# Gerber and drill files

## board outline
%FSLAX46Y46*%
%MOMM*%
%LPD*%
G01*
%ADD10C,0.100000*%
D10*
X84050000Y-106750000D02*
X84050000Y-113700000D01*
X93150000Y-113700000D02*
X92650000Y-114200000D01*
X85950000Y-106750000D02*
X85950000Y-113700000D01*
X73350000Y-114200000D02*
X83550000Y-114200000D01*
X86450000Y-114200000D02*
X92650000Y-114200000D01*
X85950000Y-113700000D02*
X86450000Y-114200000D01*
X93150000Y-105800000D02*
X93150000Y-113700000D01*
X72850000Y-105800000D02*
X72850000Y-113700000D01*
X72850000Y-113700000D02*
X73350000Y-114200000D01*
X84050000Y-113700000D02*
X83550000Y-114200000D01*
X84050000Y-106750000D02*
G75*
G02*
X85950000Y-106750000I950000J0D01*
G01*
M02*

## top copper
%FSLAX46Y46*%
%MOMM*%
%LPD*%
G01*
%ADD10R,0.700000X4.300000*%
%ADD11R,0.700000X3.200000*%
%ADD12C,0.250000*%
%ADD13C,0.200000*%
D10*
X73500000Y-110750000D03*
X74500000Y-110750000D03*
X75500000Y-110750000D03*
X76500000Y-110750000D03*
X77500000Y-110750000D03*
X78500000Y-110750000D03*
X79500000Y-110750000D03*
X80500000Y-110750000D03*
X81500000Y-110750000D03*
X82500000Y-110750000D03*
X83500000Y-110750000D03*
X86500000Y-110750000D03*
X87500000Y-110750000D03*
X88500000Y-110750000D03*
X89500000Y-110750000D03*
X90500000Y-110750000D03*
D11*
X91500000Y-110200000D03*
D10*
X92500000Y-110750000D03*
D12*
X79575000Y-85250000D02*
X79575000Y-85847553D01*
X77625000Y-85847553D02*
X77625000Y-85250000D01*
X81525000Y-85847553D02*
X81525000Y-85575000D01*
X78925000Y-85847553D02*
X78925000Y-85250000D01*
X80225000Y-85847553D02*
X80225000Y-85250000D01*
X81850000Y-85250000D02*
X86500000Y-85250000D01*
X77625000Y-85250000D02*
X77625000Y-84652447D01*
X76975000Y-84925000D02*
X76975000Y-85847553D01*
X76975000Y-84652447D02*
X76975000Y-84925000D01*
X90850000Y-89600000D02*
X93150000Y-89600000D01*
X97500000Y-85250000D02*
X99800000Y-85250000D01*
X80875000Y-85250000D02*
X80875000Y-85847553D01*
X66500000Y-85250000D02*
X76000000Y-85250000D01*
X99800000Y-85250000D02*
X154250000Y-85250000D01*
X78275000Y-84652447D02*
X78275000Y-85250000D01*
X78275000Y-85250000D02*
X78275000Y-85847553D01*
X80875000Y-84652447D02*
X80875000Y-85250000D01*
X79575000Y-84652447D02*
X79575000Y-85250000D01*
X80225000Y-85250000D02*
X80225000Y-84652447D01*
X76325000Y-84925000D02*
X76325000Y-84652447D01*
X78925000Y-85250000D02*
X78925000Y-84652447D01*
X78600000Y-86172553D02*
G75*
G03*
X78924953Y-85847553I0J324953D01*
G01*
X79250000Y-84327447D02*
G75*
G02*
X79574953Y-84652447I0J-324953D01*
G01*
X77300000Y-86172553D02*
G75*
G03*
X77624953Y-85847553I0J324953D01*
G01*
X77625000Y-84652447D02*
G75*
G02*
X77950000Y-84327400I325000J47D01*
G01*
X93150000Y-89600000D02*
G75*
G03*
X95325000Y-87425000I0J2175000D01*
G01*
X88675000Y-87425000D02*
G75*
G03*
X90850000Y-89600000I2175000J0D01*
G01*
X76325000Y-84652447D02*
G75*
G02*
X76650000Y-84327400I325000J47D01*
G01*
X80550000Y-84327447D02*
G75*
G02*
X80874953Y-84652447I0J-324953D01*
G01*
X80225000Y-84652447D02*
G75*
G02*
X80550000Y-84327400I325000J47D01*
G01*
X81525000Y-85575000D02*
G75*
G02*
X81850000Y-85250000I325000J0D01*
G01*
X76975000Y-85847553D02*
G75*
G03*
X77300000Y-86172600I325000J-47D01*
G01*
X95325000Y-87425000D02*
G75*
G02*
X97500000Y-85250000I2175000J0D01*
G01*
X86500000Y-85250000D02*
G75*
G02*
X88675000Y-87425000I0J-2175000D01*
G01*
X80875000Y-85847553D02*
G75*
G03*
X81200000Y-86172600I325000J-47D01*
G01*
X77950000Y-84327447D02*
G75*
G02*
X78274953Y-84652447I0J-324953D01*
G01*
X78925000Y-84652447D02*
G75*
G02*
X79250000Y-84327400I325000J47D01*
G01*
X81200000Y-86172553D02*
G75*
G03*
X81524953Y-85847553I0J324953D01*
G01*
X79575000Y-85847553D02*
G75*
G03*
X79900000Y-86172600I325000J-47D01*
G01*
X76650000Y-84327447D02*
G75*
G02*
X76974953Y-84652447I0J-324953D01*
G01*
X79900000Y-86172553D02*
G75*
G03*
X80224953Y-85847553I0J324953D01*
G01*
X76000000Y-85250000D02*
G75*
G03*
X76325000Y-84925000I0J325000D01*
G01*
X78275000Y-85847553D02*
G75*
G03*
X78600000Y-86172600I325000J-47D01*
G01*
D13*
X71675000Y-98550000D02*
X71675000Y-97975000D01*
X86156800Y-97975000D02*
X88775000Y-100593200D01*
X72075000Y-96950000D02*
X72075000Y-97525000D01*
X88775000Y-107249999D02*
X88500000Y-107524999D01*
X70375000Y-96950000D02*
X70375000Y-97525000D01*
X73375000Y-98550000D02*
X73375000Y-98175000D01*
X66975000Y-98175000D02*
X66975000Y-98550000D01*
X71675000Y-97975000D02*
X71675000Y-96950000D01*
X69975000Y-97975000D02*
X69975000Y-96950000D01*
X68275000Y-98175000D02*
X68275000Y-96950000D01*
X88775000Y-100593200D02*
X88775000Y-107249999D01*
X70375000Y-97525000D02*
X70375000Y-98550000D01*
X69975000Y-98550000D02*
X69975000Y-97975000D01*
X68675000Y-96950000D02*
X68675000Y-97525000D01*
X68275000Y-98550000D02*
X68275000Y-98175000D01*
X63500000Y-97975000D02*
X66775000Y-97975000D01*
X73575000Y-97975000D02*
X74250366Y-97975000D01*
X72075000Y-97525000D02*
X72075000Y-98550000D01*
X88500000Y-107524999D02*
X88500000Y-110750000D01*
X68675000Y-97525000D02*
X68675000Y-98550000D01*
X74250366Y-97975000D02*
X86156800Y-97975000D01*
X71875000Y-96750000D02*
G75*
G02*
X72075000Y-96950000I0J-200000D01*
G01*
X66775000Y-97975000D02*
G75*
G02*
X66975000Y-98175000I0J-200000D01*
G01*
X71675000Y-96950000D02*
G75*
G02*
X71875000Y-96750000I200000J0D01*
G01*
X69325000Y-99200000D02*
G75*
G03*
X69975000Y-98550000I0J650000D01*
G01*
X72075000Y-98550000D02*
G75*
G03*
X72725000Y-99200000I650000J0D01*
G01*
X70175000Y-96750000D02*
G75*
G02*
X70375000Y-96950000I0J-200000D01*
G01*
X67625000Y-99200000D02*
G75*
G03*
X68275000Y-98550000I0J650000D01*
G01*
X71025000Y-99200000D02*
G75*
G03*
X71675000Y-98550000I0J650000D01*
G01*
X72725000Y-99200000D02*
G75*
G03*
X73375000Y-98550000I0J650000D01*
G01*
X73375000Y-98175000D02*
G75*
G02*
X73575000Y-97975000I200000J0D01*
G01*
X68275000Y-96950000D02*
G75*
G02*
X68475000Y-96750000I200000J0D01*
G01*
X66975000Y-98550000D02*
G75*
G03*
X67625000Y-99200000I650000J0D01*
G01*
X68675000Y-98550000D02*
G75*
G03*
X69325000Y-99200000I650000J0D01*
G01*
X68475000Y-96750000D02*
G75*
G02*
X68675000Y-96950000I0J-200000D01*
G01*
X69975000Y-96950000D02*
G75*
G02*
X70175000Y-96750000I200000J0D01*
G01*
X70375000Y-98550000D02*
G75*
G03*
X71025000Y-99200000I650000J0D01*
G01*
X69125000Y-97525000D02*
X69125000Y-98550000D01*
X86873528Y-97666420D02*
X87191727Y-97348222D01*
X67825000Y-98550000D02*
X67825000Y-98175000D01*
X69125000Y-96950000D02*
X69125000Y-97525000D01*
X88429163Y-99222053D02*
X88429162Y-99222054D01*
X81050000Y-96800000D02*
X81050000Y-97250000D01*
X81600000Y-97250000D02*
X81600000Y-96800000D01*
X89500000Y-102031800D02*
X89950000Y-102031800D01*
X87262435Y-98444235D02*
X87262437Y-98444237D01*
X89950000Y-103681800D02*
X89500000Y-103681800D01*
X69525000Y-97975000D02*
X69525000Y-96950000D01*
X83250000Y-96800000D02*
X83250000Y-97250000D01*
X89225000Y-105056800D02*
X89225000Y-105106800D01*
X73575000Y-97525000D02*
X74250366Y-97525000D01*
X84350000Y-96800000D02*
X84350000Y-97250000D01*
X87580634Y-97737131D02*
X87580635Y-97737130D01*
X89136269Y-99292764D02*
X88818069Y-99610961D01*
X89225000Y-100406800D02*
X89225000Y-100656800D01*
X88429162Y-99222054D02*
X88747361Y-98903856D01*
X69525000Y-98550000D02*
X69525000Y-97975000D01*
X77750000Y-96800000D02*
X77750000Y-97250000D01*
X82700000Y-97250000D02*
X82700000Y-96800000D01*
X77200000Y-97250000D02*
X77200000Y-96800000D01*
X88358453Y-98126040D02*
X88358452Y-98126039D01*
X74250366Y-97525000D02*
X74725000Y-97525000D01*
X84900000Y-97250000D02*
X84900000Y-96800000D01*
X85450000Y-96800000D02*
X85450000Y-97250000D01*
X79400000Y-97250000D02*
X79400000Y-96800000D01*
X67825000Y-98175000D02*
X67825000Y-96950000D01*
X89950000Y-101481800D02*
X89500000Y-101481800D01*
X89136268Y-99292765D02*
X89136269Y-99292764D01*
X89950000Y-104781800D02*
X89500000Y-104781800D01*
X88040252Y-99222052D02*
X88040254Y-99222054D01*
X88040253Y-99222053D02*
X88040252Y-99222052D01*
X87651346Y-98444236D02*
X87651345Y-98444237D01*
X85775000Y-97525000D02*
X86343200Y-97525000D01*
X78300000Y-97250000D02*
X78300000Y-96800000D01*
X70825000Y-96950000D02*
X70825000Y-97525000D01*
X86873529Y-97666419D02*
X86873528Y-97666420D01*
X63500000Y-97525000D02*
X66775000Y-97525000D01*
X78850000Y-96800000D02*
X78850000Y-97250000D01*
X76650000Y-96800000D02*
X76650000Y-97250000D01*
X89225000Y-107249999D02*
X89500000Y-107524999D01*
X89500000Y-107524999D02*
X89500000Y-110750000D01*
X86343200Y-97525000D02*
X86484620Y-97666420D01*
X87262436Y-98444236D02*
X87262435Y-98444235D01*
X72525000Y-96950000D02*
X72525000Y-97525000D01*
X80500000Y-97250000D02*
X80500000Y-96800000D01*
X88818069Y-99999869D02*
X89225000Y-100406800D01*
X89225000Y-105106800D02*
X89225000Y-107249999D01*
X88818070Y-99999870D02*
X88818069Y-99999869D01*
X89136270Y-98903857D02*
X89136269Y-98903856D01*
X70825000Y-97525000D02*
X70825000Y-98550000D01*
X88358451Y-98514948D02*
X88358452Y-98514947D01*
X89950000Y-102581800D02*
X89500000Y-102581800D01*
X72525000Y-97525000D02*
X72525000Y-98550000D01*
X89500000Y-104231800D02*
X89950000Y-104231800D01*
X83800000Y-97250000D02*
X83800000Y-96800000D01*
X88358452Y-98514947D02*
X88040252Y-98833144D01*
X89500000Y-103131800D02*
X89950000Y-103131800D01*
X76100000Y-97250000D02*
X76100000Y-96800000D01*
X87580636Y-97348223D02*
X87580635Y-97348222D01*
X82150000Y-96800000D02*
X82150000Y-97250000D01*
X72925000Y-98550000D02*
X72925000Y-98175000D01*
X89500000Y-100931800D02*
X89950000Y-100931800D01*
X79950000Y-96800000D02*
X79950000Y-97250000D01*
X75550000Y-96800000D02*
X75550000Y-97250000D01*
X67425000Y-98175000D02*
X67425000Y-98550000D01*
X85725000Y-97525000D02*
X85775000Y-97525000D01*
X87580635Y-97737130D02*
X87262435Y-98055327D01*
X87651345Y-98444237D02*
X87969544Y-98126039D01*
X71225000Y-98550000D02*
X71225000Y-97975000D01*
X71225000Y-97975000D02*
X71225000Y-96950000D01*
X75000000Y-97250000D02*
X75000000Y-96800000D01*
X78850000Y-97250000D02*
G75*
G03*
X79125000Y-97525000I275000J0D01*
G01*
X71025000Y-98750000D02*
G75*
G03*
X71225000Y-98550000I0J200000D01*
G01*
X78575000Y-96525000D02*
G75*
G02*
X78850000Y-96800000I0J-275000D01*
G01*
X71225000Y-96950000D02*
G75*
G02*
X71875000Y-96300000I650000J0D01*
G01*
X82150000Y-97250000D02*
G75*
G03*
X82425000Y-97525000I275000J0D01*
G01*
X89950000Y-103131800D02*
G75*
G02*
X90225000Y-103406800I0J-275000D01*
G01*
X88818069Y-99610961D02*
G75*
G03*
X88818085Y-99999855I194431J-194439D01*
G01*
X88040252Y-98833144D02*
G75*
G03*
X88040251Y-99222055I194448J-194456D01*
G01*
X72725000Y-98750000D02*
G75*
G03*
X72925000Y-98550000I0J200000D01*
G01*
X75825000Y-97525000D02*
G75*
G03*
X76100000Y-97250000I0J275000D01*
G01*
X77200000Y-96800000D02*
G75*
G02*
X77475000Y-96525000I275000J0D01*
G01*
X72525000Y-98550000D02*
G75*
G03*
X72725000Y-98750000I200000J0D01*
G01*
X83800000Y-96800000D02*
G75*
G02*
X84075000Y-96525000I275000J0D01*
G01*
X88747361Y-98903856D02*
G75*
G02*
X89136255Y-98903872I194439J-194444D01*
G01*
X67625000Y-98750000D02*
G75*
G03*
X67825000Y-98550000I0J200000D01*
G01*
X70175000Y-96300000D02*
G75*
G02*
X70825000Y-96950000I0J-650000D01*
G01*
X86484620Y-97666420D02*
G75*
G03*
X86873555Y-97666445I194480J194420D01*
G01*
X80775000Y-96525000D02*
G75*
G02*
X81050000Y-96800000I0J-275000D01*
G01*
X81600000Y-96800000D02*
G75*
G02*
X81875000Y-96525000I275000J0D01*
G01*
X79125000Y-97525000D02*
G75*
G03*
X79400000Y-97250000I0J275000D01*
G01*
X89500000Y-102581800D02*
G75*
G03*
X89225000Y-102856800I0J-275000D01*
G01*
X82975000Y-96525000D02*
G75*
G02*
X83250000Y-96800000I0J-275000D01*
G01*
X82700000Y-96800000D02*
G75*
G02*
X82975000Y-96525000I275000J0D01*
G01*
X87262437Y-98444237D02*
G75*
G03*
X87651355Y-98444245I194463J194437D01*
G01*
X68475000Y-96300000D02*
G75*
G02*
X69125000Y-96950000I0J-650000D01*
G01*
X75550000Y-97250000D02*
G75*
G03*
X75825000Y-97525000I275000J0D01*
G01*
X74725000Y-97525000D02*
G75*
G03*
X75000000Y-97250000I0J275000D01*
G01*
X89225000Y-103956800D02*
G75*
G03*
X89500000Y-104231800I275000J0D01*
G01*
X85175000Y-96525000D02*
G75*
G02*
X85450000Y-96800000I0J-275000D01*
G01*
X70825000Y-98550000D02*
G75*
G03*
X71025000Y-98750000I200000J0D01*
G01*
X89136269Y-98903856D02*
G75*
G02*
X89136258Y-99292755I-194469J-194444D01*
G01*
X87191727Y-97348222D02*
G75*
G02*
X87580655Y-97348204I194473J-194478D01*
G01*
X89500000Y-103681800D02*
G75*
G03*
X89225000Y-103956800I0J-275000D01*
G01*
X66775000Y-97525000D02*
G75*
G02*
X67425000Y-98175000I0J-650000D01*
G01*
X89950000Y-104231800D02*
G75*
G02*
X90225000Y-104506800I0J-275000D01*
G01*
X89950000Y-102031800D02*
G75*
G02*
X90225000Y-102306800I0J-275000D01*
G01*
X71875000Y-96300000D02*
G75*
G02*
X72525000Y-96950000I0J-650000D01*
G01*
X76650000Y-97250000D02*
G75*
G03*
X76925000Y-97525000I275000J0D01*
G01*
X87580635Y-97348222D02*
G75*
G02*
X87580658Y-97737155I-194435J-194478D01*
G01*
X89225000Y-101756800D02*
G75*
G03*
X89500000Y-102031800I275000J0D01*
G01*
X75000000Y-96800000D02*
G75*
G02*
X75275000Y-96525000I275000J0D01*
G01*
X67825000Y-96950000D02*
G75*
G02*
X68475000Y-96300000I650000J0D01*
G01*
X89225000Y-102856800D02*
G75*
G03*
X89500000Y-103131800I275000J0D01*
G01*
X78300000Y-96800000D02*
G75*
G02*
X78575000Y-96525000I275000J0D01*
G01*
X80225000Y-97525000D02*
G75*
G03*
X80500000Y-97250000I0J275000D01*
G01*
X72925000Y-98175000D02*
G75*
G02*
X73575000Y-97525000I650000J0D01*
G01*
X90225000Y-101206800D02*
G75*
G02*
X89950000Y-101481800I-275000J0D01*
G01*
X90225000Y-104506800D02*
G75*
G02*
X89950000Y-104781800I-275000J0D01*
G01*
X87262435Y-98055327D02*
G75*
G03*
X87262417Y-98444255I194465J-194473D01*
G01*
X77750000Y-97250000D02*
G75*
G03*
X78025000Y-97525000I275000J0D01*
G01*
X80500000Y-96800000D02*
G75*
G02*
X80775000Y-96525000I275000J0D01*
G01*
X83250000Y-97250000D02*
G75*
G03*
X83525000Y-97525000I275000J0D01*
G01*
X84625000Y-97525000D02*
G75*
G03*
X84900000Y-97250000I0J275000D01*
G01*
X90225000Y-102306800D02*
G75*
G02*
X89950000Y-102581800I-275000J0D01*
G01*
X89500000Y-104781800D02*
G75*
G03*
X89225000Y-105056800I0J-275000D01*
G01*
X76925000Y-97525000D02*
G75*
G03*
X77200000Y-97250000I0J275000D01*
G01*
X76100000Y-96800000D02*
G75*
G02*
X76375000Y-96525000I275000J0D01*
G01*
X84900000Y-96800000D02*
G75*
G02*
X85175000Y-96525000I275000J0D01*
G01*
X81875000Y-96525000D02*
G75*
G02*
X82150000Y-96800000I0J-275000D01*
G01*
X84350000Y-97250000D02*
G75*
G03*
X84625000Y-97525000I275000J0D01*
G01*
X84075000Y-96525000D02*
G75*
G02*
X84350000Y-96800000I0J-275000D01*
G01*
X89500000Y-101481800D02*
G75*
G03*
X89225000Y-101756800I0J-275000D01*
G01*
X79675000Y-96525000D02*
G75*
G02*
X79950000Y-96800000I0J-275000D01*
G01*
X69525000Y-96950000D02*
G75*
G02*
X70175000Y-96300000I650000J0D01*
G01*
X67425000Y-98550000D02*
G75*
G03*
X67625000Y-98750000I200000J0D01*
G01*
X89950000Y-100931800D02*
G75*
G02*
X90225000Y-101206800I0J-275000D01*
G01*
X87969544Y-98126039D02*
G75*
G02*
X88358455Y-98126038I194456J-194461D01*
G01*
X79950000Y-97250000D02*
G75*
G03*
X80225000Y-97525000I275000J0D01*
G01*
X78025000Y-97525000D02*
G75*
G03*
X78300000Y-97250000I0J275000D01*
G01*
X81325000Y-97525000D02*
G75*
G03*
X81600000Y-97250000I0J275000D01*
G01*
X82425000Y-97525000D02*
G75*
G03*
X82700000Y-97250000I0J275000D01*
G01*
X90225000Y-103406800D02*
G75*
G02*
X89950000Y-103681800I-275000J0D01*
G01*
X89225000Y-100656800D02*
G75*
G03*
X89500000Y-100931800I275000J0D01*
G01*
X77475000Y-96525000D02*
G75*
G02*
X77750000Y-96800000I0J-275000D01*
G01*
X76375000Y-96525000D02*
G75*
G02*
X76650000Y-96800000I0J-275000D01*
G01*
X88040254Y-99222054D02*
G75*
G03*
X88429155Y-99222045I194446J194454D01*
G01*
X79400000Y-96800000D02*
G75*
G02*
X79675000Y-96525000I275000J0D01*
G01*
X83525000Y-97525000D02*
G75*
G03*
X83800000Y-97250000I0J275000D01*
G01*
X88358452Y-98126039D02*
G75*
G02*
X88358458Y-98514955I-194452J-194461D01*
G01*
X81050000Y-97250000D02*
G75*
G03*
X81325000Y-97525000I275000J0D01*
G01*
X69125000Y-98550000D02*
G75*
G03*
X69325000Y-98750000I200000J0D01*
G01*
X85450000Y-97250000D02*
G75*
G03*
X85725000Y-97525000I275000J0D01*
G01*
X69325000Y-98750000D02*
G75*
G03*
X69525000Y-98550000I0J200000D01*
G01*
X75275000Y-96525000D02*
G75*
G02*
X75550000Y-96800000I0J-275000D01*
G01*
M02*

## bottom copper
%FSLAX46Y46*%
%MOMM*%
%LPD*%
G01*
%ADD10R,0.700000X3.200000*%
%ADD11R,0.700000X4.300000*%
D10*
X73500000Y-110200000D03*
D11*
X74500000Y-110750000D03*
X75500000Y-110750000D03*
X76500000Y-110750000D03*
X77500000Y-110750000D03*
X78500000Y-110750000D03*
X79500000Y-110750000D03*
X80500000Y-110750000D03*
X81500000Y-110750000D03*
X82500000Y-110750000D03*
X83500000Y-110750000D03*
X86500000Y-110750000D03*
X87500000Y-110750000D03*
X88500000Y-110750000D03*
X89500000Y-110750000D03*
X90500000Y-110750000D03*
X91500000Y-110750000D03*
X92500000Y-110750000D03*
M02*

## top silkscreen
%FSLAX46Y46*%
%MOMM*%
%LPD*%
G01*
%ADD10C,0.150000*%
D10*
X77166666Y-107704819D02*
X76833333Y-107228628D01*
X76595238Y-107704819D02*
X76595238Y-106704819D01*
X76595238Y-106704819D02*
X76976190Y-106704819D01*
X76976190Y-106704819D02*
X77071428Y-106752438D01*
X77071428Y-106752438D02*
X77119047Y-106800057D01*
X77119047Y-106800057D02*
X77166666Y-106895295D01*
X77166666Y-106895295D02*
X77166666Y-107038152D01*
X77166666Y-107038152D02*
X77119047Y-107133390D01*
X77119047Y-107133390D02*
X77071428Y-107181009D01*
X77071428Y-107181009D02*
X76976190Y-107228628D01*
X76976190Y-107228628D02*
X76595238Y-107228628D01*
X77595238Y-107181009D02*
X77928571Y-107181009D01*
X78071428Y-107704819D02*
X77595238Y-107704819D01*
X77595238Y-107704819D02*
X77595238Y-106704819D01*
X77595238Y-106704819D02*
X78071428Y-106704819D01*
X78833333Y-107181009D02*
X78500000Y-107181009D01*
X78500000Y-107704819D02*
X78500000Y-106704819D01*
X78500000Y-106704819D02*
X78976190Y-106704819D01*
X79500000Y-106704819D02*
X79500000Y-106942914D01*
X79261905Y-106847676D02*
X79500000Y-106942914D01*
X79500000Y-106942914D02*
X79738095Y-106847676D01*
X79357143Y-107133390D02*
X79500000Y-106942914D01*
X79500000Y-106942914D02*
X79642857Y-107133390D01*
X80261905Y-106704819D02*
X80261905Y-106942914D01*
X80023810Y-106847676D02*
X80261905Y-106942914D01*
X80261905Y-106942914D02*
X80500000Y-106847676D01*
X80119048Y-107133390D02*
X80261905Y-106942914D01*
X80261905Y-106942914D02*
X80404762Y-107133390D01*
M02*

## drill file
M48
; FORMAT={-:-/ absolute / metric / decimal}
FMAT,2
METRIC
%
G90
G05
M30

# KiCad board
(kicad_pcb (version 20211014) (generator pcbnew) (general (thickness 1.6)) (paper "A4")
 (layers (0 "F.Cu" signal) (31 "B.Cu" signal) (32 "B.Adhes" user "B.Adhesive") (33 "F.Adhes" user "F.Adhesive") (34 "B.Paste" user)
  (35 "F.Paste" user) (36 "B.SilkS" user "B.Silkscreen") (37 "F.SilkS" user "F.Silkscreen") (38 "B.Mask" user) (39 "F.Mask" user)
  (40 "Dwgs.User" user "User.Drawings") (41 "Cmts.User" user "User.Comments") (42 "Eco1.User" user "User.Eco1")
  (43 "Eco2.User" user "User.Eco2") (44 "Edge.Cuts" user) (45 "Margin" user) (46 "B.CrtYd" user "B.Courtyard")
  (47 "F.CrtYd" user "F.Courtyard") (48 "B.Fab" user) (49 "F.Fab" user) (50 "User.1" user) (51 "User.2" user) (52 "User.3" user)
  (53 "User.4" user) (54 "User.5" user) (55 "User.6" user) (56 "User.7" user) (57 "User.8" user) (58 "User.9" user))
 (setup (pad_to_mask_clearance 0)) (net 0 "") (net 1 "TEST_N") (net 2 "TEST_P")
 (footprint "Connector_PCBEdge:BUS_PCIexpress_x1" (layer "F.Cu") (at 73.5 110.75)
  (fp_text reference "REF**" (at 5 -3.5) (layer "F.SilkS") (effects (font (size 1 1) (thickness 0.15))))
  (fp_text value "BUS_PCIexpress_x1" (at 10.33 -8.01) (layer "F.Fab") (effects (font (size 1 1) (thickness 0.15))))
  (fp_line (start 10.55 -4) (end 10.55 2.95) (layer "Edge.Cuts") (width 0.1))
  (fp_line (start 19.65 2.95) (end 19.15 3.45) (layer "Edge.Cuts") (width 0.1))
  (fp_line (start 12.45 -4) (end 12.45 2.95) (layer "Edge.Cuts") (width 0.1))
  (fp_line (start -0.15 3.45) (end 10.05 3.45) (layer "Edge.Cuts") (width 0.1))
  (fp_line (start 12.95 3.45) (end 19.15 3.45) (layer "Edge.Cuts") (width 0.1))
  (fp_line (start 12.45 2.95) (end 12.95 3.45) (layer "Edge.Cuts") (width 0.1))
  (fp_line (start 19.65 -4.95) (end 19.65 2.95) (layer "Edge.Cuts") (width 0.1))
  (fp_line (start -0.65 -4.95) (end -0.65 2.95) (layer "Edge.Cuts") (width 0.1))
  (fp_line (start -0.65 2.95) (end -0.15 3.45) (layer "Edge.Cuts") (width 0.1))
  (fp_line (start 10.55 2.95) (end 10.05 3.45) (layer "Edge.Cuts") (width 0.1))
  (fp_arc (start 10.55 -4) (mid 11.5 -4.95) (end 12.45 -4) (layer "Edge.Cuts") (width 0.1))
  (pad "A1" connect rect locked (at 0 -0.55) (size 0.7 3.2) (layers "B.Cu" "B.Mask"))
  (pad "A2" connect rect locked (at 1 0) (size 0.7 4.3) (layers "B.Cu" "B.Mask"))
  (pad "A3" connect rect locked (at 2 0) (size 0.7 4.3) (layers "B.Cu" "B.Mask"))
  (pad "A4" connect rect locked (at 3 0) (size 0.7 4.3) (layers "B.Cu" "B.Mask"))
  (pad "A5" connect rect locked (at 4 0) (size 0.7 4.3) (layers "B.Cu" "B.Mask"))
  (pad "A6" connect rect locked (at 5 0) (size 0.7 4.3) (layers "B.Cu" "B.Mask"))
  (pad "A7" connect rect locked (at 6 0) (size 0.7 4.3) (layers "B.Cu" "B.Mask"))
  (pad "A8" connect rect locked (at 7 0) (size 0.7 4.3) (layers "B.Cu" "B.Mask"))
  (pad "A9" connect rect locked (at 8 0) (size 0.7 4.3) (layers "B.Cu" "B.Mask"))
  (pad "A10" connect rect locked (at 9 0) (size 0.7 4.3) (layers "B.Cu" "B.Mask"))
  (pad "A11" connect rect locked (at 10 0) (size 0.7 4.3) (layers "B.Cu" "B.Mask"))
  (pad "A12" connect rect locked (at 13 0) (size 0.7 4.3) (layers "B.Cu" "B.Mask"))
  (pad "A13" connect rect locked (at 14 0) (size 0.7 4.3) (layers "B.Cu" "B.Mask"))
  (pad "A14" connect rect locked (at 15 0) (size 0.7 4.3) (layers "B.Cu" "B.Mask"))
  (pad "A15" connect rect locked (at 16 0) (size 0.7 4.3) (layers "B.Cu" "B.Mask"))
  (pad "A16" connect rect locked (at 17 0) (size 0.7 4.3) (layers "B.Cu" "B.Mask"))
  (pad "A17" connect rect locked (at 18 0) (size 0.7 4.3) (layers "B.Cu" "B.Mask"))
  (pad "A18" connect rect locked (at 19 0) (size 0.7 4.3) (layers "B.Cu" "B.Mask"))
  (pad "B1" connect rect locked (at 0 0) (size 0.7 4.3) (layers "F.Cu" "F.Mask"))
  (pad "B2" connect rect locked (at 1 0) (size 0.7 4.3) (layers "F.Cu" "F.Mask"))
  (pad "B3" connect rect locked (at 2 0) (size 0.7 4.3) (layers "F.Cu" "F.Mask"))
  (pad "B4" connect rect locked (at 3 0) (size 0.7 4.3) (layers "F.Cu" "F.Mask"))
  (pad "B5" connect rect locked (at 4 0) (size 0.7 4.3) (layers "F.Cu" "F.Mask"))
  (pad "B6" connect rect locked (at 5 0) (size 0.7 4.3) (layers "F.Cu" "F.Mask"))
  (pad "B7" connect rect locked (at 6 0) (size 0.7 4.3) (layers "F.Cu" "F.Mask"))
  (pad "B8" connect rect locked (at 7 0) (size 0.7 4.3) (layers "F.Cu" "F.Mask"))
  (pad "B9" connect rect locked (at 8 0) (size 0.7 4.3) (layers "F.Cu" "F.Mask"))
  (pad "B10" connect rect locked (at 9 0) (size 0.7 4.3) (layers "F.Cu" "F.Mask"))
  (pad "B11" connect rect locked (at 10 0) (size 0.7 4.3) (layers "F.Cu" "F.Mask"))
  (pad "B12" connect rect locked (at 13 0) (size 0.7 4.3) (layers "F.Cu" "F.Mask"))
  (pad "B13" connect rect locked (at 14 0) (size 0.7 4.3) (layers "F.Cu" "F.Mask"))
  (pad "B14" connect rect locked (at 15 0) (size 0.7 4.3) (layers "F.Cu" "F.Mask") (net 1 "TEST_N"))
  (pad "B15" connect rect locked (at 16 0) (size 0.7 4.3) (layers "F.Cu" "F.Mask") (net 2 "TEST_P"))
  (pad "B16" connect rect locked (at 17 0) (size 0.7 4.3) (layers "F.Cu" "F.Mask"))
  (pad "B17" connect rect locked (at 18 -0.55) (size 0.7 3.2) (layers "F.Cu" "F.Mask"))
  (pad "B18" connect rect locked (at 19 0) (size 0.7 4.3) (layers "F.Cu" "F.Mask")))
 (segment (start 79.575 85.25) (end 79.575 85.847553) (width 0.25) (layer "F.Cu") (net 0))
 (segment (start 77.625 85.847553) (end 77.625 85.25) (width 0.25) (layer "F.Cu") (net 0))
 (segment (start 81.525 85.847553) (end 81.525 85.575) (width 0.25) (layer "F.Cu") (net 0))
 (segment (start 78.925 85.847553) (end 78.925 85.25) (width 0.25) (layer "F.Cu") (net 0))
 (segment (start 80.225 85.847553) (end 80.225 85.25) (width 0.25) (layer "F.Cu") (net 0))
 (segment (start 81.85 85.25) (end 86.5 85.25) (width 0.25) (layer "F.Cu") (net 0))
 (segment (start 77.625 85.25) (end 77.625 84.652447) (width 0.25) (layer "F.Cu") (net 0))
 (segment (start 76.975 84.925) (end 76.975 85.847553) (width 0.25) (layer "F.Cu") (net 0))
 (segment (start 76.975 84.652447) (end 76.975 84.925) (width 0.25) (layer "F.Cu") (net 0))
 (segment (start 90.85 89.6) (end 93.15 89.6) (width 0.25) (layer "F.Cu") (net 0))
 (segment (start 97.5 85.25) (end 99.8 85.25) (width 0.25) (layer "F.Cu") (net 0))
 (segment (start 80.875 85.25) (end 80.875 85.847553) (width 0.25) (layer "F.Cu") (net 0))
 (segment (start 66.5 85.25) (end 76 85.25) (width 0.25) (layer "F.Cu") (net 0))
 (segment (start 99.8 85.25) (end 154.25 85.25) (width 0.25) (layer "F.Cu") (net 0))
 (segment (start 78.275 84.652447) (end 78.275 85.25) (width 0.25) (layer "F.Cu") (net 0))
 (segment (start 78.275 85.25) (end 78.275 85.847553) (width 0.25) (layer "F.Cu") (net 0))
 (segment (start 80.875 84.652447) (end 80.875 85.25) (width 0.25) (layer "F.Cu") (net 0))
 (segment (start 79.575 84.652447) (end 79.575 85.25) (width 0.25) (layer "F.Cu") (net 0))
 (segment (start 80.225 85.25) (end 80.225 84.652447) (width 0.25) (layer "F.Cu") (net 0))
 (segment (start 76.325 84.925) (end 76.325 84.652447) (width 0.25) (layer "F.Cu") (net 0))
 (segment (start 78.925 85.25) (end 78.925 84.652447) (width 0.25) (layer "F.Cu") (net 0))
 (arc (start 78.6 86.172553) (mid 78.82981 86.077363) (end 78.925 85.847553) (width 0.25) (layer "F.Cu") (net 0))
 (arc (start 79.25 84.327447) (mid 79.47981 84.422637) (end 79.575 84.652447) (width 0.25) (layer "F.Cu") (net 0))
 (arc (start 77.3 86.172553) (mid 77.52981 86.077363) (end 77.625 85.847553) (width 0.25) (layer "F.Cu") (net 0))
 (arc (start 77.625 84.652447) (mid 77.72019 84.422637) (end 77.95 84.327447) (width 0.25) (layer "F.Cu") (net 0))
 (arc (start 93.15 89.6) (mid 94.687957 88.962957) (end 95.325 87.425) (width 0.25) (layer "F.Cu") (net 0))
 (arc (start 88.675 87.425) (mid 89.312043 88.962957) (end 90.85 89.6) (width 0.25) (layer "F.Cu") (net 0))
 (arc (start 76.325 84.652447) (mid 76.42019 84.422637) (end 76.65 84.327447) (width 0.25) (layer "F.Cu") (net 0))
 (arc (start 80.55 84.327447) (mid 80.77981 84.422637) (end 80.875 84.652447) (width 0.25) (layer "F.Cu") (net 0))
 (arc (start 80.225 84.652447) (mid 80.32019 84.422637) (end 80.55 84.327447) (width 0.25) (layer "F.Cu") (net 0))
 (arc (start 81.525 85.575) (mid 81.62019 85.34519) (end 81.85 85.25) (width 0.25) (layer "F.Cu") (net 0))
 (arc (start 76.975 85.847553) (mid 77.07019 86.077363) (end 77.3 86.172553) (width 0.25) (layer "F.Cu") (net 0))
 (arc (start 95.325 87.425) (mid 95.962043 85.887043) (end 97.5 85.25) (width 0.25) (layer "F.Cu") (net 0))
 (arc (start 86.5 85.25) (mid 88.037957 85.887043) (end 88.675 87.425) (width 0.25) (layer "F.Cu") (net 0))
 (arc (start 80.875 85.847553) (mid 80.97019 86.077363) (end 81.2 86.172553) (width 0.25) (layer "F.Cu") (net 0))
 (arc (start 77.95 84.327447) (mid 78.17981 84.422637) (end 78.275 84.652447) (width 0.25) (layer "F.Cu") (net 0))
 (arc (start 78.925 84.652447) (mid 79.02019 84.422637) (end 79.25 84.327447) (width 0.25) (layer "F.Cu") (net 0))
 (arc (start 81.2 86.172553) (mid 81.42981 86.077363) (end 81.525 85.847553) (width 0.25) (layer "F.Cu") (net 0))
 (arc (start 79.575 85.847553) (mid 79.67019 86.077363) (end 79.9 86.172553) (width 0.25) (layer "F.Cu") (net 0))
 (arc (start 76.65 84.327447) (mid 76.87981 84.422637) (end 76.975 84.652447) (width 0.25) (layer "F.Cu") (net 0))
 (arc (start 79.9 86.172553) (mid 80.12981 86.077363) (end 80.225 85.847553) (width 0.25) (layer "F.Cu") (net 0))
 (arc (start 76 85.25) (mid 76.22981 85.15481) (end 76.325 84.925) (width 0.25) (layer "F.Cu") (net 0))
 (arc (start 78.275 85.847553) (mid 78.37019 86.077363) (end 78.6 86.172553) (width 0.25) (layer "F.Cu") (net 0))
 (segment (start 71.675 98.55) (end 71.675 97.975) (width 0.2) (layer "F.Cu") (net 1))
 (segment (start 86.1568 97.975) (end 88.775 100.5932) (width 0.2) (layer "F.Cu") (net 1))
 (segment (start 72.075 96.95) (end 72.075 97.525) (width 0.2) (layer "F.Cu") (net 1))
 (segment (start 88.775 107.249999) (end 88.5 107.524999) (width 0.2) (layer "F.Cu") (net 1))
 (segment (start 70.375 96.95) (end 70.375 97.525) (width 0.2) (layer "F.Cu") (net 1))
 (segment (start 73.375 98.55) (end 73.375 98.175) (width 0.2) (layer "F.Cu") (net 1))
 (segment (start 66.975 98.175) (end 66.975 98.55) (width 0.2) (layer "F.Cu") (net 1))
 (segment (start 71.675 97.975) (end 71.675 96.95) (width 0.2) (layer "F.Cu") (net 1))
 (segment (start 69.975 97.975) (end 69.975 96.95) (width 0.2) (layer "F.Cu") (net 1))
 (segment (start 68.275 98.175) (end 68.275 96.95) (width 0.2) (layer "F.Cu") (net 1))
 (segment (start 88.775 100.5932) (end 88.775 107.249999) (width 0.2) (layer "F.Cu") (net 1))
 (segment (start 70.375 97.525) (end 70.375 98.55) (width 0.2) (layer "F.Cu") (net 1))
 (segment (start 69.975 98.55) (end 69.975 97.975) (width 0.2) (layer "F.Cu") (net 1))
 (segment (start 68.675 96.95) (end 68.675 97.525) (width 0.2) (layer "F.Cu") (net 1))
 (segment (start 68.275 98.55) (end 68.275 98.175) (width 0.2) (layer "F.Cu") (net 1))
 (segment (start 63.5 97.975) (end 66.775 97.975) (width 0.2) (layer "F.Cu") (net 1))
 (segment (start 73.575 97.975) (end 74.250366 97.975) (width 0.2) (layer "F.Cu") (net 1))
 (segment (start 72.075 97.525) (end 72.075 98.55) (width 0.2) (layer "F.Cu") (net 1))
 (segment (start 88.5 107.524999) (end 88.5 110.75) (width 0.2) (layer "F.Cu") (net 1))
 (segment (start 68.675 97.525) (end 68.675 98.55) (width 0.2) (layer "F.Cu") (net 1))
 (segment (start 74.250366 97.975) (end 86.1568 97.975) (width 0.2) (layer "F.Cu") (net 1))
 (arc (start 71.875 96.75) (mid 72.016421 96.808579) (end 72.075 96.95) (width 0.2) (layer "F.Cu") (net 1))
 (arc (start 66.775 97.975) (mid 66.916421 98.033579) (end 66.975 98.175) (width 0.2) (layer "F.Cu") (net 1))
 (arc (start 71.675 96.95) (mid 71.733579 96.808579) (end 71.875 96.75) (width 0.2) (layer "F.Cu") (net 1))
 (arc (start 69.325 99.2) (mid 69.784619 99.009619) (end 69.975 98.55) (width 0.2) (layer "F.Cu") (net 1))
 (arc (start 72.075 98.55) (mid 72.265381 99.009619) (end 72.725 99.2) (width 0.2) (layer "F.Cu") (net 1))
 (arc (start 70.175 96.75) (mid 70.316421 96.808579) (end 70.375 96.95) (width 0.2) (layer "F.Cu") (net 1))
 (arc (start 67.625 99.2) (mid 68.084619 99.009619) (end 68.275 98.55) (width 0.2) (layer "F.Cu") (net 1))
 (arc (start 71.025 99.2) (mid 71.484619 99.009619) (end 71.675 98.55) (width 0.2) (layer "F.Cu") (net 1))
 (arc (start 72.725 99.2) (mid 73.184619 99.009619) (end 73.375 98.55) (width 0.2) (layer "F.Cu") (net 1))
 (arc (start 73.375 98.175) (mid 73.433579 98.033579) (end 73.575 97.975) (width 0.2) (layer "F.Cu") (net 1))
 (arc (start 68.275 96.95) (mid 68.333579 96.808579) (end 68.475 96.75) (width 0.2) (layer "F.Cu") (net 1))
 (arc (start 66.975 98.55) (mid 67.165381 99.009619) (end 67.625 99.2) (width 0.2) (layer "F.Cu") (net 1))
 (arc (start 68.675 98.55) (mid 68.865381 99.009619) (end 69.325 99.2) (width 0.2) (layer "F.Cu") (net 1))
 (arc (start 68.475 96.75) (mid 68.616421 96.808579) (end 68.675 96.95) (width 0.2) (layer "F.Cu") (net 1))
 (arc (start 69.975 96.95) (mid 70.033579 96.808579) (end 70.175 96.75) (width 0.2) (layer "F.Cu") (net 1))
 (arc (start 70.375 98.55) (mid 70.565381 99.009619) (end 71.025 99.2) (width 0.2) (layer "F.Cu") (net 1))
 (segment (start 69.125 97.525) (end 69.125 98.55) (width 0.2) (layer "F.Cu") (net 2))
 (segment (start 86.873528 97.66642) (end 87.191727 97.348222) (width 0.2) (layer "F.Cu") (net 2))
 (segment (start 67.825 98.55) (end 67.825 98.175) (width 0.2) (layer "F.Cu") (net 2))
 (segment (start 69.125 96.95) (end 69.125 97.525) (width 0.2) (layer "F.Cu") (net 2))
 (segment (start 88.429163 99.222053) (end 88.429162 99.222054) (width 0.2) (layer "F.Cu") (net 2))
 (segment (start 81.05 96.8) (end 81.05 97.25) (width 0.2) (layer "F.Cu") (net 2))
 (segment (start 81.6 97.25) (end 81.6 96.8) (width 0.2) (layer "F.Cu") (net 2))
 (segment (start 89.5 102.0318) (end 89.95 102.0318) (width 0.2) (layer "F.Cu") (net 2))
 (segment (start 87.262435 98.444235) (end 87.262437 98.444237) (width 0.2) (layer "F.Cu") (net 2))
 (segment (start 89.95 103.6818) (end 89.5 103.6818) (width 0.2) (layer "F.Cu") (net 2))
 (segment (start 69.525 97.975) (end 69.525 96.95) (width 0.2) (layer "F.Cu") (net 2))
 (segment (start 83.25 96.8) (end 83.25 97.25) (width 0.2) (layer "F.Cu") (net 2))
 (segment (start 89.225 105.0568) (end 89.225 105.1068) (width 0.2) (layer "F.Cu") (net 2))
 (segment (start 73.575 97.525) (end 74.250366 97.525) (width 0.2) (layer "F.Cu") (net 2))
 (segment (start 84.35 96.8) (end 84.35 97.25) (width 0.2) (layer "F.Cu") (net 2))
 (segment (start 87.580634 97.737131) (end 87.580635 97.73713) (width 0.2) (layer "F.Cu") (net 2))
 (segment (start 89.136269 99.292764) (end 88.818069 99.610961) (width 0.2) (layer "F.Cu") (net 2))
 (segment (start 89.225 100.4068) (end 89.225 100.6568) (width 0.2) (layer "F.Cu") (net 2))
 (segment (start 88.429162 99.222054) (end 88.747361 98.903856) (width 0.2) (layer "F.Cu") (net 2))
 (segment (start 69.525 98.55) (end 69.525 97.975) (width 0.2) (layer "F.Cu") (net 2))
 (segment (start 77.75 96.8) (end 77.75 97.25) (width 0.2) (layer "F.Cu") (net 2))
 (segment (start 82.7 97.25) (end 82.7 96.8) (width 0.2) (layer "F.Cu") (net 2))
 (segment (start 77.2 97.25) (end 77.2 96.8) (width 0.2) (layer "F.Cu") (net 2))
 (segment (start 88.358453 98.12604) (end 88.358452 98.126039) (width 0.2) (layer "F.Cu") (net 2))
 (segment (start 74.250366 97.525) (end 74.725 97.525) (width 0.2) (layer "F.Cu") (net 2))
 (segment (start 84.9 97.25) (end 84.9 96.8) (width 0.2) (layer "F.Cu") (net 2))
 (segment (start 85.45 96.8) (end 85.45 97.25) (width 0.2) (layer "F.Cu") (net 2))
 (segment (start 79.4 97.25) (end 79.4 96.8) (width 0.2) (layer "F.Cu") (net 2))
 (segment (start 67.825 98.175) (end 67.825 96.95) (width 0.2) (layer "F.Cu") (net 2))
 (segment (start 89.95 101.4818) (end 89.5 101.4818) (width 0.2) (layer "F.Cu") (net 2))
 (segment (start 89.136268 99.292765) (end 89.136269 99.292764) (width 0.2) (layer "F.Cu") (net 2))
 (segment (start 89.95 104.7818) (end 89.5 104.7818) (width 0.2) (layer "F.Cu") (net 2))
 (segment (start 88.040252 99.222052) (end 88.040254 99.222054) (width 0.2) (layer "F.Cu") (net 2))
 (segment (start 88.040253 99.222053) (end 88.040252 99.222052) (width 0.2) (layer "F.Cu") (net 2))
 (segment (start 87.651346 98.444236) (end 87.651345 98.444237) (width 0.2) (layer "F.Cu") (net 2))
 (segment (start 85.775 97.525) (end 86.3432 97.525) (width 0.2) (layer "F.Cu") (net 2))
 (segment (start 78.3 97.25) (end 78.3 96.8) (width 0.2) (layer "F.Cu") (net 2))
 (segment (start 70.825 96.95) (end 70.825 97.525) (width 0.2) (layer "F.Cu") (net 2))
 (segment (start 86.873529 97.666419) (end 86.873528 97.66642) (width 0.2) (layer "F.Cu") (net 2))
 (segment (start 63.5 97.525) (end 66.775 97.525) (width 0.2) (layer "F.Cu") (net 2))
 (segment (start 78.85 96.8) (end 78.85 97.25) (width 0.2) (layer "F.Cu") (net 2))
 (segment (start 76.65 96.8) (end 76.65 97.25) (width 0.2) (layer "F.Cu") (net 2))
 (segment (start 89.225 107.249999) (end 89.5 107.524999) (width 0.2) (layer "F.Cu") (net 2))
 (segment (start 89.5 107.524999) (end 89.5 110.75) (width 0.2) (layer "F.Cu") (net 2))
 (segment (start 86.3432 97.525) (end 86.48462 97.66642) (width 0.2) (layer "F.Cu") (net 2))
 (segment (start 87.262436 98.444236) (end 87.262435 98.444235) (width 0.2) (layer "F.Cu") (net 2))
 (segment (start 72.525 96.95) (end 72.525 97.525) (width 0.2) (layer "F.Cu") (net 2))
 (segment (start 80.5 97.25) (end 80.5 96.8) (width 0.2) (layer "F.Cu") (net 2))
 (segment (start 88.818069 99.999869) (end 89.225 100.4068) (width 0.2) (layer "F.Cu") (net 2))
 (segment (start 89.225 105.1068) (end 89.225 107.249999) (width 0.2) (layer "F.Cu") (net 2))
 (segment (start 88.81807 99.99987) (end 88.818069 99.999869) (width 0.2) (layer "F.Cu") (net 2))
 (segment (start 89.13627 98.903857) (end 89.136269 98.903856) (width 0.2) (layer "F.Cu") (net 2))
 (segment (start 70.825 97.525) (end 70.825 98.55) (width 0.2) (layer "F.Cu") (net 2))
 (segment (start 88.358451 98.514948) (end 88.358452 98.514947) (width 0.2) (layer "F.Cu") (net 2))
 (segment (start 89.95 102.5818) (end 89.5 102.5818) (width 0.2) (layer "F.Cu") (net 2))
 (segment (start 72.525 97.525) (end 72.525 98.55) (width 0.2) (layer "F.Cu") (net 2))
 (segment (start 89.5 104.2318) (end 89.95 104.2318) (width 0.2) (layer "F.Cu") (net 2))
 (segment (start 83.8 97.25) (end 83.8 96.8) (width 0.2) (layer "F.Cu") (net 2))
 (segment (start 88.358452 98.514947) (end 88.040252 98.833144) (width 0.2) (layer "F.Cu") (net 2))
 (segment (start 89.5 103.1318) (end 89.95 103.1318) (width 0.2) (layer "F.Cu") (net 2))
 (segment (start 76.1 97.25) (end 76.1 96.8) (width 0.2) (layer "F.Cu") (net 2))
 (segment (start 87.580636 97.348223) (end 87.580635 97.348222) (width 0.2) (layer "F.Cu") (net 2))
 (segment (start 82.15 96.8) (end 82.15 97.25) (width 0.2) (layer "F.Cu") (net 2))
 (segment (start 72.925 98.55) (end 72.925 98.175) (width 0.2) (layer "F.Cu") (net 2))
 (segment (start 89.5 100.9318) (end 89.95 100.9318) (width 0.2) (layer "F.Cu") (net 2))
 (segment (start 79.95 96.8) (end 79.95 97.25) (width 0.2) (layer "F.Cu") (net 2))
 (segment (start 75.55 96.8) (end 75.55 97.25) (width 0.2) (layer "F.Cu") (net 2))
 (segment (start 67.425 98.175) (end 67.425 98.55) (width 0.2) (layer "F.Cu") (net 2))
 (segment (start 85.725 97.525) (end 85.775 97.525) (width 0.2) (layer "F.Cu") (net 2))
 (segment (start 87.580635 97.73713) (end 87.262435 98.055327) (width 0.2) (layer "F.Cu") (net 2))
 (segment (start 87.651345 98.444237) (end 87.969544 98.126039) (width 0.2) (layer "F.Cu") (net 2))
 (segment (start 71.225 98.55) (end 71.225 97.975) (width 0.2) (layer "F.Cu") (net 2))
 (segment (start 71.225 97.975) (end 71.225 96.95) (width 0.2) (layer "F.Cu") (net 2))
 (segment (start 75 97.25) (end 75 96.8) (width 0.2) (layer "F.Cu") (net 2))
 (arc (start 78.85 97.25) (mid 78.930546 97.444454) (end 79.125 97.525) (width 0.2) (layer "F.Cu") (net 2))
 (arc (start 71.025 98.75) (mid 71.166421 98.691421) (end 71.225 98.55) (width 0.2) (layer "F.Cu") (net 2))
 (arc (start 78.575 96.525) (mid 78.769454 96.605546) (end 78.85 96.8) (width 0.2) (layer "F.Cu") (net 2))
 (arc (start 71.225 96.95) (mid 71.415381 96.490381) (end 71.875 96.3) (width 0.2) (layer "F.Cu") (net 2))
 (arc (start 82.15 97.25) (mid 82.230546 97.444454) (end 82.425 97.525) (width 0.2) (layer "F.Cu") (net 2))
 (arc (start 89.95 103.1318) (mid 90.144454 103.212346) (end 90.225 103.4068) (width 0.2) (layer "F.Cu") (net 2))
 (arc (start 88.818069 99.610961) (mid 88.737524 99.805416) (end 88.81807 99.99987) (width 0.2) (layer "F.Cu") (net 2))
 (arc (start 88.040252 98.833144) (mid 87.959707 99.027599) (end 88.040253 99.222053) (width 0.2) (layer "F.Cu") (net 2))
 (arc (start 72.725 98.75) (mid 72.866421 98.691421) (end 72.925 98.55) (width 0.2) (layer "F.Cu") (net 2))
 (arc (start 75.825 97.525) (mid 76.019454 97.444454) (end 76.1 97.25) (width 0.2) (layer "F.Cu") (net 2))
 (arc (start 77.2 96.8) (mid 77.280546 96.605546) (end 77.475 96.525) (width 0.2) (layer "F.Cu") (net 2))
 (arc (start 72.525 98.55) (mid 72.583579 98.691421) (end 72.725 98.75) (width 0.2) (layer "F.Cu") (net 2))
 (arc (start 83.8 96.8) (mid 83.880546 96.605546) (end 84.075 96.525) (width 0.2) (layer "F.Cu") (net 2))
 (arc (start 88.747361 98.903856) (mid 88.941816 98.823311) (end 89.13627 98.903857) (width 0.2) (layer "F.Cu") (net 2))
 (arc (start 67.625 98.75) (mid 67.766421 98.691421) (end 67.825 98.55) (width 0.2) (layer "F.Cu") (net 2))
 (arc (start 70.175 96.3) (mid 70.634619 96.490381) (end 70.825 96.95) (width 0.2) (layer "F.Cu") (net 2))
 (arc (start 86.48462 97.66642) (mid 86.679075 97.746965) (end 86.873529 97.666419) (width 0.2) (layer "F.Cu") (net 2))
 (arc (start 80.775 96.525) (mid 80.969454 96.605546) (end 81.05 96.8) (width 0.2) (layer "F.Cu") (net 2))
 (arc (start 81.6 96.8) (mid 81.680546 96.605546) (end 81.875 96.525) (width 0.2) (layer "F.Cu") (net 2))
 (arc (start 79.125 97.525) (mid 79.319454 97.444454) (end 79.4 97.25) (width 0.2) (layer "F.Cu") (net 2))
 (arc (start 89.5 102.5818) (mid 89.305546 102.662346) (end 89.225 102.8568) (width 0.2) (layer "F.Cu") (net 2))
 (arc (start 82.975 96.525) (mid 83.169454 96.605546) (end 83.25 96.8) (width 0.2) (layer "F.Cu") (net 2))
 (arc (start 82.7 96.8) (mid 82.780546 96.605546) (end 82.975 96.525) (width 0.2) (layer "F.Cu") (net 2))
 (arc (start 87.262437 98.444237) (mid 87.456892 98.524782) (end 87.651346 98.444236) (width 0.2) (layer "F.Cu") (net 2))
 (arc (start 68.475 96.3) (mid 68.934619 96.490381) (end 69.125 96.95) (width 0.2) (layer "F.Cu") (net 2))
 (arc (start 75.55 97.25) (mid 75.630546 97.444454) (end 75.825 97.525) (width 0.2) (layer "F.Cu") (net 2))
 (arc (start 74.725 97.525) (mid 74.919454 97.444454) (end 75 97.25) (width 0.2) (layer "F.Cu") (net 2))
 (arc (start 89.225 103.9568) (mid 89.305546 104.151254) (end 89.5 104.2318) (width 0.2) (layer "F.Cu") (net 2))
 (arc (start 85.175 96.525) (mid 85.369454 96.605546) (end 85.45 96.8) (width 0.2) (layer "F.Cu") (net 2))
 (arc (start 70.825 98.55) (mid 70.883579 98.691421) (end 71.025 98.75) (width 0.2) (layer "F.Cu") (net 2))
 (arc (start 89.136269 98.903856) (mid 89.216814 99.098311) (end 89.136268 99.292765) (width 0.2) (layer "F.Cu") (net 2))
 (arc (start 87.191727 97.348222) (mid 87.386182 97.267677) (end 87.580636 97.348223) (width 0.2) (layer "F.Cu") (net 2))
 (arc (start 89.5 103.6818) (mid 89.305546 103.762346) (end 89.225 103.9568) (width 0.2) (layer "F.Cu") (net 2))
 (arc (start 66.775 97.525) (mid 67.234619 97.715381) (end 67.425 98.175) (width 0.2) (layer "F.Cu") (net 2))
 (arc (start 89.95 104.2318) (mid 90.144454 104.312346) (end 90.225 104.5068) (width 0.2) (layer "F.Cu") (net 2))
 (arc (start 89.95 102.0318) (mid 90.144454 102.112346) (end 90.225 102.3068) (width 0.2) (layer "F.Cu") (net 2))
 (arc (start 71.875 96.3) (mid 72.334619 96.490381) (end 72.525 96.95) (width 0.2) (layer "F.Cu") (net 2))
 (arc (start 76.65 97.25) (mid 76.730546 97.444454) (end 76.925 97.525) (width 0.2) (layer "F.Cu") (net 2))
 (arc (start 87.580635 97.348222) (mid 87.66118 97.542677) (end 87.580634 97.737131) (width 0.2) (layer "F.Cu") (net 2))
 (arc (start 89.225 101.7568) (mid 89.305546 101.951254) (end 89.5 102.0318) (width 0.2) (layer "F.Cu") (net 2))
 (arc (start 75 96.8) (mid 75.080546 96.605546) (end 75.275 96.525) (width 0.2) (layer "F.Cu") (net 2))
 (arc (start 67.825 96.95) (mid 68.015381 96.490381) (end 68.475 96.3) (width 0.2) (layer "F.Cu") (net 2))
 (arc (start 89.225 102.8568) (mid 89.305546 103.051254) (end 89.5 103.1318) (width 0.2) (layer "F.Cu") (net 2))
 (arc (start 78.3 96.8) (mid 78.380546 96.605546) (end 78.575 96.525) (width 0.2) (layer "F.Cu") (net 2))
 (arc (start 80.225 97.525) (mid 80.419454 97.444454) (end 80.5 97.25) (width 0.2) (layer "F.Cu") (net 2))
 (arc (start 72.925 98.175) (mid 73.115381 97.715381) (end 73.575 97.525) (width 0.2) (layer "F.Cu") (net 2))
 (arc (start 90.225 101.2068) (mid 90.144454 101.401254) (end 89.95 101.4818) (width 0.2) (layer "F.Cu") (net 2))
 (arc (start 90.225 104.5068) (mid 90.144454 104.701254) (end 89.95 104.7818) (width 0.2) (layer "F.Cu") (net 2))
 (arc (start 87.262435 98.055327) (mid 87.18189 98.249782) (end 87.262436 98.444236) (width 0.2) (layer "F.Cu") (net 2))
 (arc (start 77.75 97.25) (mid 77.830546 97.444454) (end 78.025 97.525) (width 0.2) (layer "F.Cu") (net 2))
 (arc (start 80.5 96.8) (mid 80.580546 96.605546) (end 80.775 96.525) (width 0.2) (layer "F.Cu") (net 2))
 (arc (start 83.25 97.25) (mid 83.330546 97.444454) (end 83.525 97.525) (width 0.2) (layer "F.Cu") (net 2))
 (arc (start 84.625 97.525) (mid 84.819454 97.444454) (end 84.9 97.25) (width 0.2) (layer "F.Cu") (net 2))
 (arc (start 90.225 102.3068) (mid 90.144454 102.501254) (end 89.95 102.5818) (width 0.2) (layer "F.Cu") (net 2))
 (arc (start 89.5 104.7818) (mid 89.305546 104.862346) (end 89.225 105.0568) (width 0.2) (layer "F.Cu") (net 2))
 (arc (start 76.925 97.525) (mid 77.119454 97.444454) (end 77.2 97.25) (width 0.2) (layer "F.Cu") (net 2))
 (arc (start 76.1 96.8) (mid 76.180546 96.605546) (end 76.375 96.525) (width 0.2) (layer "F.Cu") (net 2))
 (arc (start 84.9 96.8) (mid 84.980546 96.605546) (end 85.175 96.525) (width 0.2) (layer "F.Cu") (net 2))
 (arc (start 81.875 96.525) (mid 82.069454 96.605546) (end 82.15 96.8) (width 0.2) (layer "F.Cu") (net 2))
 (arc (start 84.35 97.25) (mid 84.430546 97.444454) (end 84.625 97.525) (width 0.2) (layer "F.Cu") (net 2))
 (arc (start 84.075 96.525) (mid 84.269454 96.605546) (end 84.35 96.8) (width 0.2) (layer "F.Cu") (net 2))
 (arc (start 89.5 101.4818) (mid 89.305546 101.562346) (end 89.225 101.7568) (width 0.2) (layer "F.Cu") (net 2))
 (arc (start 79.675 96.525) (mid 79.869454 96.605546) (end 79.95 96.8) (width 0.2) (layer "F.Cu") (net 2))
 (arc (start 69.525 96.95) (mid 69.715381 96.490381) (end 70.175 96.3) (width 0.2) (layer "F.Cu") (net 2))
 (arc (start 67.425 98.55) (mid 67.483579 98.691421) (end 67.625 98.75) (width 0.2) (layer "F.Cu") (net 2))
 (arc (start 89.95 100.9318) (mid 90.144454 101.012346) (end 90.225 101.2068) (width 0.2) (layer "F.Cu") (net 2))
 (arc (start 87.969544 98.126039) (mid 88.163999 98.045494) (end 88.358453 98.12604) (width 0.2) (layer "F.Cu") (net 2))
 (arc (start 79.95 97.25) (mid 80.030546 97.444454) (end 80.225 97.525) (width 0.2) (layer "F.Cu") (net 2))
 (arc (start 78.025 97.525) (mid 78.219454 97.444454) (end 78.3 97.25) (width 0.2) (layer "F.Cu") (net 2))
 (arc (start 81.325 97.525) (mid 81.519454 97.444454) (end 81.6 97.25) (width 0.2) (layer "F.Cu") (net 2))
 (arc (start 82.425 97.525) (mid 82.619454 97.444454) (end 82.7 97.25) (width 0.2) (layer "F.Cu") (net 2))
 (arc (start 90.225 103.4068) (mid 90.144454 103.601254) (end 89.95 103.6818) (width 0.2) (layer "F.Cu") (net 2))
 (arc (start 89.225 100.6568) (mid 89.305546 100.851254) (end 89.5 100.9318) (width 0.2) (layer "F.Cu") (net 2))
 (arc (start 77.475 96.525) (mid 77.669454 96.605546) (end 77.75 96.8) (width 0.2) (layer "F.Cu") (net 2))
 (arc (start 76.375 96.525) (mid 76.569454 96.605546) (end 76.65 96.8) (width 0.2) (layer "F.Cu") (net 2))
 (arc (start 88.040254 99.222054) (mid 88.234709 99.302599) (end 88.429163 99.222053) (width 0.2) (layer "F.Cu") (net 2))
 (arc (start 79.4 96.8) (mid 79.480546 96.605546) (end 79.675 96.525) (width 0.2) (layer "F.Cu") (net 2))
 (arc (start 83.525 97.525) (mid 83.719454 97.444454) (end 83.8 97.25) (width 0.2) (layer "F.Cu") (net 2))
 (arc (start 88.358452 98.126039) (mid 88.438997 98.320494) (end 88.358451 98.514948) (width 0.2) (layer "F.Cu") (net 2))
 (arc (start 81.05 97.25) (mid 81.130546 97.444454) (end 81.325 97.525) (width 0.2) (layer "F.Cu") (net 2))
 (arc (start 69.125 98.55) (mid 69.183579 98.691421) (end 69.325 98.75) (width 0.2) (layer "F.Cu") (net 2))
 (arc (start 85.45 97.25) (mid 85.530546 97.444454) (end 85.725 97.525) (width 0.2) (layer "F.Cu") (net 2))
 (arc (start 69.325 98.75) (mid 69.466421 98.691421) (end 69.525 98.55) (width 0.2) (layer "F.Cu") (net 2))
 (arc (start 75.275 96.525) (mid 75.469454 96.605546) (end 75.55 96.8) (width 0.2) (layer "F.Cu") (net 2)))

